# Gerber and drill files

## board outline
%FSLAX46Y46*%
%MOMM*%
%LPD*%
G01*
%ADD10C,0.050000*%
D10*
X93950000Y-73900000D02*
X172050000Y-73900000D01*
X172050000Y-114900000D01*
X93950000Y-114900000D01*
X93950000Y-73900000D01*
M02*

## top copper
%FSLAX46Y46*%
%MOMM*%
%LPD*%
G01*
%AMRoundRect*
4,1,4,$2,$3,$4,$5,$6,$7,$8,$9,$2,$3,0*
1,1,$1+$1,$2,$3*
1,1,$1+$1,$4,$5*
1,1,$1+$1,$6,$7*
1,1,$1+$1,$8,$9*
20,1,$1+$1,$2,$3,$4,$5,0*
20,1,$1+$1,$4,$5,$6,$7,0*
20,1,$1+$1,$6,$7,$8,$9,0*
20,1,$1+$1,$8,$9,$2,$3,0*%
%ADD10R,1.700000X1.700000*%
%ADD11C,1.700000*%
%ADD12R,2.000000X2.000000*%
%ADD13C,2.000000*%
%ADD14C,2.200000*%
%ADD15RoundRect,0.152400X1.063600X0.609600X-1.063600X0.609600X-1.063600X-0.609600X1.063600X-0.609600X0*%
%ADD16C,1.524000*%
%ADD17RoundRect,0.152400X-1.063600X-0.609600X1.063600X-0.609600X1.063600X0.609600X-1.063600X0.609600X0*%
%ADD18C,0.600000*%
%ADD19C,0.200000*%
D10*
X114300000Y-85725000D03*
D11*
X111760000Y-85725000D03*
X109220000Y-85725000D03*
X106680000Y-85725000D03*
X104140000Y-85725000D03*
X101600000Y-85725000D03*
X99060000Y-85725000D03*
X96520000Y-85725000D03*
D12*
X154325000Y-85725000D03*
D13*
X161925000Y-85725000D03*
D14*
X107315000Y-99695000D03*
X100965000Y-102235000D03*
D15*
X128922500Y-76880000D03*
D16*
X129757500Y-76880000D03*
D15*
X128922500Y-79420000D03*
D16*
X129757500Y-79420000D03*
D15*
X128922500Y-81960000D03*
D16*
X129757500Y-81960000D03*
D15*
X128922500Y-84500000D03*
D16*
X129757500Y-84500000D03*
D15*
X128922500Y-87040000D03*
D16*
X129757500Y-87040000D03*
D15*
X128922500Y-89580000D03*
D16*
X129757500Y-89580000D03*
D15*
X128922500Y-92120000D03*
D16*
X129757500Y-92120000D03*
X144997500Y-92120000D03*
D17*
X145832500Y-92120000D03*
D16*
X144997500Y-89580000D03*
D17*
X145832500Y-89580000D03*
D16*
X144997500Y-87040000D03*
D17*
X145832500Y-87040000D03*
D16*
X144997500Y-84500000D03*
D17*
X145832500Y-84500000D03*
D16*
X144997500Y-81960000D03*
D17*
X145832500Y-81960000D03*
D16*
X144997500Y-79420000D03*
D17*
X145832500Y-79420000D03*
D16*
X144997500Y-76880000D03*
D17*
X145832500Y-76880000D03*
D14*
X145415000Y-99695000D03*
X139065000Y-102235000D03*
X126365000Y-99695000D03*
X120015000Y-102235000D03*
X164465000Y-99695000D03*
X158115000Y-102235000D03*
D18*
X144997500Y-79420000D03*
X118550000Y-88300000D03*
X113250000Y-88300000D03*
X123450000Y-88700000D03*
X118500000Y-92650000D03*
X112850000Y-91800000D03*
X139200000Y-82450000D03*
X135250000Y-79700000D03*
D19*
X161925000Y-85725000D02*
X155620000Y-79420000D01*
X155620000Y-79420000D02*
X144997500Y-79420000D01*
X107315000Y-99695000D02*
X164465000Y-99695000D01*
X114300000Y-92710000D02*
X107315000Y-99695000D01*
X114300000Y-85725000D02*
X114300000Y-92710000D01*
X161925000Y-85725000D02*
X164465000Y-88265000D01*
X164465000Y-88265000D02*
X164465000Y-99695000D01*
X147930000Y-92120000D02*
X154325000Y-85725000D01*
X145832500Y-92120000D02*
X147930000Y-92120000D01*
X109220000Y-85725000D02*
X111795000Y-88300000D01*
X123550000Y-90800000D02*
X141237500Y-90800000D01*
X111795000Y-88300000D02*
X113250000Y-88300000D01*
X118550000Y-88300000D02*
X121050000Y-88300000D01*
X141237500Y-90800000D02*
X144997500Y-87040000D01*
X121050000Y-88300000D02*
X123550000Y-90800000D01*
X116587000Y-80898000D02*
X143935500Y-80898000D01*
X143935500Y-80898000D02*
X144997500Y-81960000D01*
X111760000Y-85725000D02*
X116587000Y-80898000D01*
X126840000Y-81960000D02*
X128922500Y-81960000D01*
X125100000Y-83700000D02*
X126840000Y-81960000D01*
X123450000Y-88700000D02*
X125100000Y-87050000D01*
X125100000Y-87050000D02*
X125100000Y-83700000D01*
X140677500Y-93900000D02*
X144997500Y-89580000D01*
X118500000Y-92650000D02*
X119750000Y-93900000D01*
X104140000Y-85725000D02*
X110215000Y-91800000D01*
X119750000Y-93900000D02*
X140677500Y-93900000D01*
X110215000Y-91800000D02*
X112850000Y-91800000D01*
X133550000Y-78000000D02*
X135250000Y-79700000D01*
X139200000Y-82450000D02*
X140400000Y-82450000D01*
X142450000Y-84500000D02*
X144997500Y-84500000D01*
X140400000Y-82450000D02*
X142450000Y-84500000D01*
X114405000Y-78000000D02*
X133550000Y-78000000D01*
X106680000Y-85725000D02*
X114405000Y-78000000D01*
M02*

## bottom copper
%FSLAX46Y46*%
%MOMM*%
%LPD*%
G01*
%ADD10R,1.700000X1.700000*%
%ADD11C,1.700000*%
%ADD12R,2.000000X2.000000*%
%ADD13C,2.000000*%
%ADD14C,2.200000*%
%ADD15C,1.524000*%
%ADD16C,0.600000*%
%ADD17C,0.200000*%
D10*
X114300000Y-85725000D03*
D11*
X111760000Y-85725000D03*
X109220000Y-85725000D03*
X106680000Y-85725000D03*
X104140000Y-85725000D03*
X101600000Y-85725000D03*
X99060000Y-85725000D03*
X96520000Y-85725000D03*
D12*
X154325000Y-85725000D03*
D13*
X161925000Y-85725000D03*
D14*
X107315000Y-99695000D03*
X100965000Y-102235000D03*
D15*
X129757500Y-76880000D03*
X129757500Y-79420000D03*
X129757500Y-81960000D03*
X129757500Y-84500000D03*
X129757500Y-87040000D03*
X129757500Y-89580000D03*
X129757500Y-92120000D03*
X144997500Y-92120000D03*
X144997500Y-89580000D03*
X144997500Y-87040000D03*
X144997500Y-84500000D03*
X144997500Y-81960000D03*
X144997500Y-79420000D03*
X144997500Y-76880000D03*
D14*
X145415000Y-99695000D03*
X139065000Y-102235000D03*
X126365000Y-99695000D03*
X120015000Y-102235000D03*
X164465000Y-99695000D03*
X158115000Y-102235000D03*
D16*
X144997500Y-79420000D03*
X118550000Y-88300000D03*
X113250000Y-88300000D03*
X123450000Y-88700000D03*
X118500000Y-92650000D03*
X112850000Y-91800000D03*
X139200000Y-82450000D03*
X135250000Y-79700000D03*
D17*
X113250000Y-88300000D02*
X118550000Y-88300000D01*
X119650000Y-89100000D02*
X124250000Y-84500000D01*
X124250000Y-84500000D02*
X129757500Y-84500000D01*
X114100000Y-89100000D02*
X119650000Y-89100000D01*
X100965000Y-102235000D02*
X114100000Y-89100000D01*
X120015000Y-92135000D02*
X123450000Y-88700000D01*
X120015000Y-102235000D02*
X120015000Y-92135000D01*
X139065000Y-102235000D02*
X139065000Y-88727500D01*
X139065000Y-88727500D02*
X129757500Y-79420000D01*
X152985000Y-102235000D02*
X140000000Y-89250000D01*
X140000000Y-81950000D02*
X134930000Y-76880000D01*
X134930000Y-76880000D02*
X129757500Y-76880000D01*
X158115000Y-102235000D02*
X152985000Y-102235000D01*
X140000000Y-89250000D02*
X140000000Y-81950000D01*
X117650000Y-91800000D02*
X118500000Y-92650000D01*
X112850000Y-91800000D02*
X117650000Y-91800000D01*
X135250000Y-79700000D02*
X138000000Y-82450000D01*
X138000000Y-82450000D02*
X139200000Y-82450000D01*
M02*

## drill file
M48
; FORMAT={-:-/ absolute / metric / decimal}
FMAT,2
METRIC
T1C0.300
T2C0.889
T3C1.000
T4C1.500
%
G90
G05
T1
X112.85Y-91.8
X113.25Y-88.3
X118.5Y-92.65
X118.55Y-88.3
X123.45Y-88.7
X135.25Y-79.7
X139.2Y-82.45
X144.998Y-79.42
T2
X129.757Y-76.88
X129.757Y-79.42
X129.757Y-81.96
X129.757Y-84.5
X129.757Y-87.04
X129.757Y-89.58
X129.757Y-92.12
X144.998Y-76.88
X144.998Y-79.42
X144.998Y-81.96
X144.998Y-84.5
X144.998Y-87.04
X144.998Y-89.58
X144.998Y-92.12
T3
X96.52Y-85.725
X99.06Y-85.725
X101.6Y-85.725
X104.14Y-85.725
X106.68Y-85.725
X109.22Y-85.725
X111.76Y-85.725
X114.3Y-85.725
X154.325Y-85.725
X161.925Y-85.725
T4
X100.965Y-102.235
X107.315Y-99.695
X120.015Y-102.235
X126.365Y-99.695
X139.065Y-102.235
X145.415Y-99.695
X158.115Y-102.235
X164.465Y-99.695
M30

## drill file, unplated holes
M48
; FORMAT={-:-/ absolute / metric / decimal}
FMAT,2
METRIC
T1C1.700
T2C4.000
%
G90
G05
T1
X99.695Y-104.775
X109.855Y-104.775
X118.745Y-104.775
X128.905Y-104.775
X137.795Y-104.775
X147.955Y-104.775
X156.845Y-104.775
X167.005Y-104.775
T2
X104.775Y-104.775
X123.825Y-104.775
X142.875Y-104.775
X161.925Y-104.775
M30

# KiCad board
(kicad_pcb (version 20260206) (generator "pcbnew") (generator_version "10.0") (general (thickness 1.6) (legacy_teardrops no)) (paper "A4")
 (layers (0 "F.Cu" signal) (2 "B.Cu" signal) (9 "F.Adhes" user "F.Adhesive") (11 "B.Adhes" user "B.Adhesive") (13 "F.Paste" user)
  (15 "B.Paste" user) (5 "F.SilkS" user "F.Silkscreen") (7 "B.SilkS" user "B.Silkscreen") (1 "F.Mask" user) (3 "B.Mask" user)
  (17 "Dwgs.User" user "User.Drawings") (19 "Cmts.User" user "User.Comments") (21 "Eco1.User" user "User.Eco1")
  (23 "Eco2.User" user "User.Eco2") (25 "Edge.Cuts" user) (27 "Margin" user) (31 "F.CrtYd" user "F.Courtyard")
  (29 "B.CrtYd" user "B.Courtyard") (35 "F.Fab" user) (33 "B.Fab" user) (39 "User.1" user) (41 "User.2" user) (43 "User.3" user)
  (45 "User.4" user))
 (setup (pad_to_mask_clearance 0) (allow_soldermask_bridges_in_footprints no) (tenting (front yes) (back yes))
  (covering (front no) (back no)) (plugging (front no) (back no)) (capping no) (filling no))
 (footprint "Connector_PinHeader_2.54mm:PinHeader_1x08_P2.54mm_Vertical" (layer "F.Cu") (at 114.3 85.725 -90)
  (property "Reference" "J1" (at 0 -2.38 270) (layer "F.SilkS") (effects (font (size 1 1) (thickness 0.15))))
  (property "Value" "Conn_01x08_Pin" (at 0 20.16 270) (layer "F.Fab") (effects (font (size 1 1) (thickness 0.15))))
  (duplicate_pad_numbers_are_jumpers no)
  (pad "1" thru_hole rect (at 0 0 270) (size 1.7 1.7) (drill 1) (layers "*.Cu" "*.Mask") (remove_unused_layers no) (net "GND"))
  (pad "2" thru_hole circle (at 0 2.54 270) (size 1.7 1.7) (drill 1) (layers "*.Cu" "*.Mask") (remove_unused_layers no) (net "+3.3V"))
  (pad "3" thru_hole circle (at 0 5.08 270) (size 1.7 1.7) (drill 1) (layers "*.Cu" "*.Mask") (remove_unused_layers no)
   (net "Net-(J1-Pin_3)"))
  (pad "4" thru_hole circle (at 0 7.62 270) (size 1.7 1.7) (drill 1) (layers "*.Cu" "*.Mask") (remove_unused_layers no)
   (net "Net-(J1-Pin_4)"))
  (pad "5" thru_hole circle (at 0 10.16 270) (size 1.7 1.7) (drill 1) (layers "*.Cu" "*.Mask") (remove_unused_layers no)
   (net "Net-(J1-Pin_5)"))
  (pad "6" thru_hole circle (at 0 12.7 270) (size 1.7 1.7) (drill 1) (layers "*.Cu" "*.Mask") (remove_unused_layers no)
   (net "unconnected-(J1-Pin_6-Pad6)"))
  (pad "7" thru_hole circle (at 0 15.24 270) (size 1.7 1.7) (drill 1) (layers "*.Cu" "*.Mask") (remove_unused_layers no)
   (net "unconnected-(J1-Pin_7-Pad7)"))
  (pad "8" thru_hole circle (at 0 17.78 270) (size 1.7 1.7) (drill 1) (layers "*.Cu" "*.Mask") (remove_unused_layers no)
   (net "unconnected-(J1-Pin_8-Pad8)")))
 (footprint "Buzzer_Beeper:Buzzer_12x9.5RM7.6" (layer "F.Cu") (at 154.325 85.725)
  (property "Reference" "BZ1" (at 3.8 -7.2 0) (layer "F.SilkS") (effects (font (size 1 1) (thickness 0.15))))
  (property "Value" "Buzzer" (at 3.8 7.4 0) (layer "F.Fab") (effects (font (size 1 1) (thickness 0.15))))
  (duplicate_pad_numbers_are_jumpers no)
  (pad "1" thru_hole rect (at 0 0) (size 2 2) (drill 1) (layers "*.Cu" "*.Mask") (remove_unused_layers no) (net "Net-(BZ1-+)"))
  (pad "2" thru_hole circle (at 7.6 0) (size 2 2) (drill 1) (layers "*.Cu" "*.Mask") (remove_unused_layers no) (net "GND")))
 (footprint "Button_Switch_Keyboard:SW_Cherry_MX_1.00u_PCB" (layer "F.Cu") (at 107.315 99.695)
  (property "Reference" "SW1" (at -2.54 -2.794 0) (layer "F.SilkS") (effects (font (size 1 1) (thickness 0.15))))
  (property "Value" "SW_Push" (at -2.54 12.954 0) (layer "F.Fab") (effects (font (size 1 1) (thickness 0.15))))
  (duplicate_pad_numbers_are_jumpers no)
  (pad "" np_thru_hole circle (at -7.62 5.08) (size 1.7 1.7) (drill 1.7) (layers "*.Cu" "*.Mask"))
  (pad "" np_thru_hole circle (at -2.54 5.08) (size 4 4) (drill 4) (layers "*.Cu" "*.Mask"))
  (pad "" np_thru_hole circle (at 2.54 5.08) (size 1.7 1.7) (drill 1.7) (layers "*.Cu" "*.Mask"))
  (pad "1" thru_hole circle (at 0 0) (size 2.2 2.2) (drill 1.5) (layers "*.Cu" "*.Mask") (remove_unused_layers no) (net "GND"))
  (pad "2" thru_hole circle (at -6.35 2.54) (size 2.2 2.2) (drill 1.5) (layers "*.Cu" "*.Mask") (remove_unused_layers no)
   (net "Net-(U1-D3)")))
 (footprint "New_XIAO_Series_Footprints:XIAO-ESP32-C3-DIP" (layer "F.Cu") (at 137.3775 84.5 90)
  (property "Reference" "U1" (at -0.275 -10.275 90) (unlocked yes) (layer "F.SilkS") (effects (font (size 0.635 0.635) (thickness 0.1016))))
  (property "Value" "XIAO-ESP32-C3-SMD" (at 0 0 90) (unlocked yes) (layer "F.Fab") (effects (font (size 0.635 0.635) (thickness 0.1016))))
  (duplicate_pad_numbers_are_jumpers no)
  (pad "1" smd roundrect (at 7.62 -8.455 180) (size 2.432 1.524) (layers "F.Cu" "F.Mask") (roundrect_rratio 0.1) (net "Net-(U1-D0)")
   (thermal_bridge_angle 45))
  (pad "1" thru_hole circle (at 7.62 -7.62 180) (size 1.524 1.524) (drill 0.889) (layers "*.Cu" "*.Mask") (remove_unused_layers no)
   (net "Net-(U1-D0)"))
  (pad "2" smd roundrect (at 5.08 -8.455 180) (size 2.432 1.524) (layers "F.Cu" "F.Mask") (roundrect_rratio 0.1) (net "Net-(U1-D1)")
   (thermal_bridge_angle 45))
  (pad "2" thru_hole circle (at 5.08 -7.62 180) (size 1.524 1.524) (drill 0.889) (layers "*.Cu" "*.Mask") (remove_unused_layers no)
   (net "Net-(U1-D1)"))
  (pad "3" smd roundrect (at 2.54 -8.455 180) (size 2.432 1.524) (layers "F.Cu" "F.Mask") (roundrect_rratio 0.1) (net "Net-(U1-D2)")
   (thermal_bridge_angle 45))
  (pad "3" thru_hole circle (at 2.54 -7.62 180) (size 1.524 1.524) (drill 0.889) (layers "*.Cu" "*.Mask") (remove_unused_layers no)
   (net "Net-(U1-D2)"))
  (pad "4" smd roundrect (at 0 -8.455 180) (size 2.432 1.524) (layers "F.Cu" "F.Mask") (roundrect_rratio 0.1) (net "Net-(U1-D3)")
   (thermal_bridge_angle 45))
  (pad "4" thru_hole circle (at 0 -7.62 180) (size 1.524 1.524) (drill 0.889) (layers "*.Cu" "*.Mask") (remove_unused_layers no)
   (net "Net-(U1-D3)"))
  (pad "5" smd roundrect (at -2.54 -8.455 180) (size 2.432 1.524) (layers "F.Cu" "F.Mask") (roundrect_rratio 0.1)
   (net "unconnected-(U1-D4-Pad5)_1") (thermal_bridge_angle 45))
  (pad "5" thru_hole circle (at -2.54 -7.62 180) (size 1.524 1.524) (drill 0.889) (layers "*.Cu" "*.Mask") (remove_unused_layers no)
   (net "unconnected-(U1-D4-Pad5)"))
  (pad "6" smd roundrect (at -5.08 -8.455 180) (size 2.432 1.524) (layers "F.Cu" "F.Mask") (roundrect_rratio 0.1)
   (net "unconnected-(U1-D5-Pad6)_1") (thermal_bridge_angle 45))
  (pad "6" thru_hole circle (at -5.08 -7.62 180) (size 1.524 1.524) (drill 0.889) (layers "*.Cu" "*.Mask") (remove_unused_layers no)
   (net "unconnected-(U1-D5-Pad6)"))
  (pad "7" smd roundrect (at -7.62 -8.455 180) (size 2.432 1.524) (layers "F.Cu" "F.Mask") (roundrect_rratio 0.1)
   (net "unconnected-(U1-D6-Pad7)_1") (thermal_bridge_angle 45))
  (pad "7" thru_hole circle (at -7.62 -7.62 180) (size 1.524 1.524) (drill 0.889) (layers "*.Cu" "*.Mask") (remove_unused_layers no)
   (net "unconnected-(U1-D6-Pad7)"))
  (pad "8" thru_hole circle (at -7.62 7.62) (size 1.524 1.524) (drill 0.889) (layers "*.Cu" "*.Mask") (remove_unused_layers no)
   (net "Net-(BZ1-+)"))
  (pad "8" smd roundrect (at -7.62 8.455) (size 2.432 1.524) (layers "F.Cu" "F.Mask") (roundrect_rratio 0.1) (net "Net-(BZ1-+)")
   (thermal_bridge_angle 45))
  (pad "9" thru_hole circle (at -5.08 7.62) (size 1.524 1.524) (drill 0.889) (layers "*.Cu" "*.Mask") (remove_unused_layers no)
   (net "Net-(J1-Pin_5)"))
  (pad "9" smd roundrect (at -5.08 8.455) (size 2.432 1.524) (layers "F.Cu" "F.Mask") (roundrect_rratio 0.1) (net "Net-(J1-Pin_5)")
   (thermal_bridge_angle 45))
  (pad "10" thru_hole circle (at -2.54 7.62) (size 1.524 1.524) (drill 0.889) (layers "*.Cu" "*.Mask") (remove_unused_layers no)
   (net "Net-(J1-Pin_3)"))
  (pad "10" smd roundrect (at -2.54 8.455) (size 2.432 1.524) (layers "F.Cu" "F.Mask") (roundrect_rratio 0.1) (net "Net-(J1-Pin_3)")
   (thermal_bridge_angle 45))
  (pad "11" thru_hole circle (at 0 7.62) (size 1.524 1.524) (drill 0.889) (layers "*.Cu" "*.Mask") (remove_unused_layers no)
   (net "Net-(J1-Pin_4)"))
  (pad "11" smd roundrect (at 0 8.455) (size 2.432 1.524) (layers "F.Cu" "F.Mask") (roundrect_rratio 0.1) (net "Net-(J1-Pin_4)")
   (thermal_bridge_angle 45))
  (pad "12" thru_hole circle (at 2.54 7.62) (size 1.524 1.524) (drill 0.889) (layers "*.Cu" "*.Mask") (remove_unused_layers no)
   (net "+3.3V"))
  (pad "12" smd roundrect (at 2.54 8.455) (size 2.432 1.524) (layers "F.Cu" "F.Mask") (roundrect_rratio 0.1) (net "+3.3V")
   (thermal_bridge_angle 45))
  (pad "13" thru_hole circle (at 5.08 7.62) (size 1.524 1.524) (drill 0.889) (layers "*.Cu" "*.Mask") (remove_unused_layers no) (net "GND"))
  (pad "13" smd roundrect (at 5.08 8.455) (size 2.432 1.524) (layers "F.Cu" "F.Mask") (roundrect_rratio 0.1) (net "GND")
   (thermal_bridge_angle 45))
  (pad "14" thru_hole circle (at 7.62 7.62) (size 1.524 1.524) (drill 0.889) (layers "*.Cu" "*.Mask") (remove_unused_layers no)
   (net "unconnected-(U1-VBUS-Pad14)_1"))
  (pad "14" smd roundrect (at 7.62 8.455) (size 2.432 1.524) (layers "F.Cu" "F.Mask") (roundrect_rratio 0.1)
   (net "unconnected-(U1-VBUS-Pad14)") (thermal_bridge_angle 45)))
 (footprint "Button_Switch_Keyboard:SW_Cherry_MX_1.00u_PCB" (layer "F.Cu") (at 145.415 99.695)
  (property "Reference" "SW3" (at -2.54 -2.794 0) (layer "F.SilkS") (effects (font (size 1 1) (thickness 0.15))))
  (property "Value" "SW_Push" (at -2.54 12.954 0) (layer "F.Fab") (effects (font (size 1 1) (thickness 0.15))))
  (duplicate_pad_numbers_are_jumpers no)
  (pad "" np_thru_hole circle (at -7.62 5.08) (size 1.7 1.7) (drill 1.7) (layers "*.Cu" "*.Mask"))
  (pad "" np_thru_hole circle (at -2.54 5.08) (size 4 4) (drill 4) (layers "*.Cu" "*.Mask"))
  (pad "" np_thru_hole circle (at 2.54 5.08) (size 1.7 1.7) (drill 1.7) (layers "*.Cu" "*.Mask"))
  (pad "1" thru_hole circle (at 0 0) (size 2.2 2.2) (drill 1.5) (layers "*.Cu" "*.Mask") (remove_unused_layers no) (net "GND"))
  (pad "2" thru_hole circle (at -6.35 2.54) (size 2.2 2.2) (drill 1.5) (layers "*.Cu" "*.Mask") (remove_unused_layers no)
   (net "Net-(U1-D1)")))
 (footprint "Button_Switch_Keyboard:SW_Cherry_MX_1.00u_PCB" (layer "F.Cu") (at 126.365 99.695)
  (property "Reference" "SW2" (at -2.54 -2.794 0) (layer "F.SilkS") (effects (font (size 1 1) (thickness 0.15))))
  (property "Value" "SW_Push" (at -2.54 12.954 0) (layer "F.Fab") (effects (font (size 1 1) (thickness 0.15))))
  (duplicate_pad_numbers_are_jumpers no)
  (pad "" np_thru_hole circle (at -7.62 5.08) (size 1.7 1.7) (drill 1.7) (layers "*.Cu" "*.Mask"))
  (pad "" np_thru_hole circle (at -2.54 5.08) (size 4 4) (drill 4) (layers "*.Cu" "*.Mask"))
  (pad "" np_thru_hole circle (at 2.54 5.08) (size 1.7 1.7) (drill 1.7) (layers "*.Cu" "*.Mask"))
  (pad "1" thru_hole circle (at 0 0) (size 2.2 2.2) (drill 1.5) (layers "*.Cu" "*.Mask") (remove_unused_layers no) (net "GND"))
  (pad "2" thru_hole circle (at -6.35 2.54) (size 2.2 2.2) (drill 1.5) (layers "*.Cu" "*.Mask") (remove_unused_layers no)
   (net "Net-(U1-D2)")))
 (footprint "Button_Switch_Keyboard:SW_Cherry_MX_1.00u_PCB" (layer "F.Cu") (at 164.465 99.695)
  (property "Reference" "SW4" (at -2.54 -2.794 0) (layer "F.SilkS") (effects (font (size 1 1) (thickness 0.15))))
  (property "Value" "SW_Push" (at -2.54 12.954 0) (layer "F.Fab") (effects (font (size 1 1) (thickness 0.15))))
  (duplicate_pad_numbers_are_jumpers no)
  (pad "" np_thru_hole circle (at -7.62 5.08) (size 1.7 1.7) (drill 1.7) (layers "*.Cu" "*.Mask"))
  (pad "" np_thru_hole circle (at -2.54 5.08) (size 4 4) (drill 4) (layers "*.Cu" "*.Mask"))
  (pad "" np_thru_hole circle (at 2.54 5.08) (size 1.7 1.7) (drill 1.7) (layers "*.Cu" "*.Mask"))
  (pad "1" thru_hole circle (at 0 0) (size 2.2 2.2) (drill 1.5) (layers "*.Cu" "*.Mask") (remove_unused_layers no) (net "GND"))
  (pad "2" thru_hole circle (at -6.35 2.54) (size 2.2 2.2) (drill 1.5) (layers "*.Cu" "*.Mask") (remove_unused_layers no)
   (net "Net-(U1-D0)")))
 (gr_rect (start 93.95 73.9) (end 172.05 114.9) (stroke (width 0.05) (type default)) (fill no) (layer "Edge.Cuts"))
 (segment (start 161.925 85.725) (end 155.62 79.42) (width 0.2) (layer "F.Cu") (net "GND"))
 (segment (start 155.62 79.42) (end 144.9975 79.42) (width 0.2) (layer "F.Cu") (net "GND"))
 (segment (start 107.315 99.695) (end 164.465 99.695) (width 0.2) (layer "F.Cu") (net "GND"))
 (segment (start 114.3 92.71) (end 107.315 99.695) (width 0.2) (layer "F.Cu") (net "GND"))
 (segment (start 114.3 85.725) (end 114.3 92.71) (width 0.2) (layer "F.Cu") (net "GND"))
 (segment (start 161.925 85.725) (end 164.465 88.265) (width 0.2) (layer "F.Cu") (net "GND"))
 (segment (start 164.465 88.265) (end 164.465 99.695) (width 0.2) (layer "F.Cu") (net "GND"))
 (via (at 144.9975 79.42) (size 0.6) (drill 0.3) (layers "F.Cu" "B.Cu") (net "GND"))
 (segment (start 116.587 80.898) (end 143.9355 80.898) (width 0.2) (layer "F.Cu") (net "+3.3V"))
 (segment (start 143.9355 80.898) (end 144.9975 81.96) (width 0.2) (layer "F.Cu") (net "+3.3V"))
 (segment (start 111.76 85.725) (end 116.587 80.898) (width 0.2) (layer "F.Cu") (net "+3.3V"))
 (segment (start 109.22 85.725) (end 111.795 88.3) (width 0.2) (layer "F.Cu") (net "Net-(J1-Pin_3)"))
 (segment (start 123.55 90.8) (end 141.2375 90.8) (width 0.2) (layer "F.Cu") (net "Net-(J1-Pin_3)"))
 (segment (start 111.795 88.3) (end 113.25 88.3) (width 0.2) (layer "F.Cu") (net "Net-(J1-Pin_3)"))
 (segment (start 118.55 88.3) (end 121.05 88.3) (width 0.2) (layer "F.Cu") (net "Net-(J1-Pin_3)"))
 (segment (start 141.2375 90.8) (end 144.9975 87.04) (width 0.2) (layer "F.Cu") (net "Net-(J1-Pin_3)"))
 (segment (start 121.05 88.3) (end 123.55 90.8) (width 0.2) (layer "F.Cu") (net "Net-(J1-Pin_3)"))
 (via (at 118.55 88.3) (size 0.6) (drill 0.3) (layers "F.Cu" "B.Cu") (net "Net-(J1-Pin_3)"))
 (via (at 113.25 88.3) (size 0.6) (drill 0.3) (layers "F.Cu" "B.Cu") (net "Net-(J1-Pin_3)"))
 (segment (start 113.25 88.3) (end 118.55 88.3) (width 0.2) (layer "B.Cu") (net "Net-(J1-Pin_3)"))
 (segment (start 133.55 78) (end 135.25 79.7) (width 0.2) (layer "F.Cu") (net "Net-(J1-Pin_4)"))
 (segment (start 139.2 82.45) (end 140.4 82.45) (width 0.2) (layer "F.Cu") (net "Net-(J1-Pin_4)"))
 (segment (start 142.45 84.5) (end 144.9975 84.5) (width 0.2) (layer "F.Cu") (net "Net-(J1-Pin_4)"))
 (segment (start 140.4 82.45) (end 142.45 84.5) (width 0.2) (layer "F.Cu") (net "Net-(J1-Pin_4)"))
 (segment (start 114.405 78) (end 133.55 78) (width 0.2) (layer "F.Cu") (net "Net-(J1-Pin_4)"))
 (segment (start 106.68 85.725) (end 114.405 78) (width 0.2) (layer "F.Cu") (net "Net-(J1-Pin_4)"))
 (via (at 139.2 82.45) (size 0.6) (drill 0.3) (layers "F.Cu" "B.Cu") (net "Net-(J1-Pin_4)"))
 (via (at 135.25 79.7) (size 0.6) (drill 0.3) (layers "F.Cu" "B.Cu") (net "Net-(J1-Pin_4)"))
 (segment (start 135.25 79.7) (end 138 82.45) (width 0.2) (layer "B.Cu") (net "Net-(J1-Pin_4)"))
 (segment (start 138 82.45) (end 139.2 82.45) (width 0.2) (layer "B.Cu") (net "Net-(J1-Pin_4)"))
 (segment (start 140.6775 93.9) (end 144.9975 89.58) (width 0.2) (layer "F.Cu") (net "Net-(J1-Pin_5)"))
 (segment (start 118.5 92.65) (end 119.75 93.9) (width 0.2) (layer "F.Cu") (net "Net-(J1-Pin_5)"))
 (segment (start 104.14 85.725) (end 110.215 91.8) (width 0.2) (layer "F.Cu") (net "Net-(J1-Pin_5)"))
 (segment (start 119.75 93.9) (end 140.6775 93.9) (width 0.2) (layer "F.Cu") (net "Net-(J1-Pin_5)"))
 (segment (start 110.215 91.8) (end 112.85 91.8) (width 0.2) (layer "F.Cu") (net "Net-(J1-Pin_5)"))
 (via (at 118.5 92.65) (size 0.6) (drill 0.3) (layers "F.Cu" "B.Cu") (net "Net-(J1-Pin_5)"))
 (via (at 112.85 91.8) (size 0.6) (drill 0.3) (layers "F.Cu" "B.Cu") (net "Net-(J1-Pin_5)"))
 (segment (start 117.65 91.8) (end 118.5 92.65) (width 0.2) (layer "B.Cu") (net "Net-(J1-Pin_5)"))
 (segment (start 112.85 91.8) (end 117.65 91.8) (width 0.2) (layer "B.Cu") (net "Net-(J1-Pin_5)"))
 (segment (start 147.93 92.12) (end 154.325 85.725) (width 0.2) (layer "F.Cu") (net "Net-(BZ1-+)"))
 (segment (start 145.8325 92.12) (end 147.93 92.12) (width 0.2) (layer "F.Cu") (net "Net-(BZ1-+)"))
 (segment (start 119.65 89.1) (end 124.25 84.5) (width 0.2) (layer "B.Cu") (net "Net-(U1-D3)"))
 (segment (start 124.25 84.5) (end 129.7575 84.5) (width 0.2) (layer "B.Cu") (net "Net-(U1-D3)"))
 (segment (start 114.1 89.1) (end 119.65 89.1) (width 0.2) (layer "B.Cu") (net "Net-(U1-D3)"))
 (segment (start 100.965 102.235) (end 114.1 89.1) (width 0.2) (layer "B.Cu") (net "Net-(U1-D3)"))
 (segment (start 152.985 102.235) (end 140 89.25) (width 0.2) (layer "B.Cu") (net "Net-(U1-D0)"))
 (segment (start 140 81.95) (end 134.93 76.88) (width 0.2) (layer "B.Cu") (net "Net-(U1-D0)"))
 (segment (start 134.93 76.88) (end 129.7575 76.88) (width 0.2) (layer "B.Cu") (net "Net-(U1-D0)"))
 (segment (start 158.115 102.235) (end 152.985 102.235) (width 0.2) (layer "B.Cu") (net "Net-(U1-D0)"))
 (segment (start 140 89.25) (end 140 81.95) (width 0.2) (layer "B.Cu") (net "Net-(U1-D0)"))
 (segment (start 139.065 102.235) (end 139.065 88.7275) (width 0.2) (layer "B.Cu") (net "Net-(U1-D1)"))
 (segment (start 139.065 88.7275) (end 129.7575 79.42) (width 0.2) (layer "B.Cu") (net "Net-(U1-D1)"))
 (segment (start 126.84 81.96) (end 128.9225 81.96) (width 0.2) (layer "F.Cu") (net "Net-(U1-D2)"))
 (segment (start 125.1 83.7) (end 126.84 81.96) (width 0.2) (layer "F.Cu") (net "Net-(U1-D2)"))
 (segment (start 123.45 88.7) (end 125.1 87.05) (width 0.2) (layer "F.Cu") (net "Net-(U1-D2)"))
 (segment (start 125.1 87.05) (end 125.1 83.7) (width 0.2) (layer "F.Cu") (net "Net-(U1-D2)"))
 (via (at 123.45 88.7) (size 0.6) (drill 0.3) (layers "F.Cu" "B.Cu") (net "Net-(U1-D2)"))
 (segment (start 120.015 92.135) (end 123.45 88.7) (width 0.2) (layer "B.Cu") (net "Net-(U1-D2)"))
 (segment (start 120.015 102.235) (end 120.015 92.135) (width 0.2) (layer "B.Cu") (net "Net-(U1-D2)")))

